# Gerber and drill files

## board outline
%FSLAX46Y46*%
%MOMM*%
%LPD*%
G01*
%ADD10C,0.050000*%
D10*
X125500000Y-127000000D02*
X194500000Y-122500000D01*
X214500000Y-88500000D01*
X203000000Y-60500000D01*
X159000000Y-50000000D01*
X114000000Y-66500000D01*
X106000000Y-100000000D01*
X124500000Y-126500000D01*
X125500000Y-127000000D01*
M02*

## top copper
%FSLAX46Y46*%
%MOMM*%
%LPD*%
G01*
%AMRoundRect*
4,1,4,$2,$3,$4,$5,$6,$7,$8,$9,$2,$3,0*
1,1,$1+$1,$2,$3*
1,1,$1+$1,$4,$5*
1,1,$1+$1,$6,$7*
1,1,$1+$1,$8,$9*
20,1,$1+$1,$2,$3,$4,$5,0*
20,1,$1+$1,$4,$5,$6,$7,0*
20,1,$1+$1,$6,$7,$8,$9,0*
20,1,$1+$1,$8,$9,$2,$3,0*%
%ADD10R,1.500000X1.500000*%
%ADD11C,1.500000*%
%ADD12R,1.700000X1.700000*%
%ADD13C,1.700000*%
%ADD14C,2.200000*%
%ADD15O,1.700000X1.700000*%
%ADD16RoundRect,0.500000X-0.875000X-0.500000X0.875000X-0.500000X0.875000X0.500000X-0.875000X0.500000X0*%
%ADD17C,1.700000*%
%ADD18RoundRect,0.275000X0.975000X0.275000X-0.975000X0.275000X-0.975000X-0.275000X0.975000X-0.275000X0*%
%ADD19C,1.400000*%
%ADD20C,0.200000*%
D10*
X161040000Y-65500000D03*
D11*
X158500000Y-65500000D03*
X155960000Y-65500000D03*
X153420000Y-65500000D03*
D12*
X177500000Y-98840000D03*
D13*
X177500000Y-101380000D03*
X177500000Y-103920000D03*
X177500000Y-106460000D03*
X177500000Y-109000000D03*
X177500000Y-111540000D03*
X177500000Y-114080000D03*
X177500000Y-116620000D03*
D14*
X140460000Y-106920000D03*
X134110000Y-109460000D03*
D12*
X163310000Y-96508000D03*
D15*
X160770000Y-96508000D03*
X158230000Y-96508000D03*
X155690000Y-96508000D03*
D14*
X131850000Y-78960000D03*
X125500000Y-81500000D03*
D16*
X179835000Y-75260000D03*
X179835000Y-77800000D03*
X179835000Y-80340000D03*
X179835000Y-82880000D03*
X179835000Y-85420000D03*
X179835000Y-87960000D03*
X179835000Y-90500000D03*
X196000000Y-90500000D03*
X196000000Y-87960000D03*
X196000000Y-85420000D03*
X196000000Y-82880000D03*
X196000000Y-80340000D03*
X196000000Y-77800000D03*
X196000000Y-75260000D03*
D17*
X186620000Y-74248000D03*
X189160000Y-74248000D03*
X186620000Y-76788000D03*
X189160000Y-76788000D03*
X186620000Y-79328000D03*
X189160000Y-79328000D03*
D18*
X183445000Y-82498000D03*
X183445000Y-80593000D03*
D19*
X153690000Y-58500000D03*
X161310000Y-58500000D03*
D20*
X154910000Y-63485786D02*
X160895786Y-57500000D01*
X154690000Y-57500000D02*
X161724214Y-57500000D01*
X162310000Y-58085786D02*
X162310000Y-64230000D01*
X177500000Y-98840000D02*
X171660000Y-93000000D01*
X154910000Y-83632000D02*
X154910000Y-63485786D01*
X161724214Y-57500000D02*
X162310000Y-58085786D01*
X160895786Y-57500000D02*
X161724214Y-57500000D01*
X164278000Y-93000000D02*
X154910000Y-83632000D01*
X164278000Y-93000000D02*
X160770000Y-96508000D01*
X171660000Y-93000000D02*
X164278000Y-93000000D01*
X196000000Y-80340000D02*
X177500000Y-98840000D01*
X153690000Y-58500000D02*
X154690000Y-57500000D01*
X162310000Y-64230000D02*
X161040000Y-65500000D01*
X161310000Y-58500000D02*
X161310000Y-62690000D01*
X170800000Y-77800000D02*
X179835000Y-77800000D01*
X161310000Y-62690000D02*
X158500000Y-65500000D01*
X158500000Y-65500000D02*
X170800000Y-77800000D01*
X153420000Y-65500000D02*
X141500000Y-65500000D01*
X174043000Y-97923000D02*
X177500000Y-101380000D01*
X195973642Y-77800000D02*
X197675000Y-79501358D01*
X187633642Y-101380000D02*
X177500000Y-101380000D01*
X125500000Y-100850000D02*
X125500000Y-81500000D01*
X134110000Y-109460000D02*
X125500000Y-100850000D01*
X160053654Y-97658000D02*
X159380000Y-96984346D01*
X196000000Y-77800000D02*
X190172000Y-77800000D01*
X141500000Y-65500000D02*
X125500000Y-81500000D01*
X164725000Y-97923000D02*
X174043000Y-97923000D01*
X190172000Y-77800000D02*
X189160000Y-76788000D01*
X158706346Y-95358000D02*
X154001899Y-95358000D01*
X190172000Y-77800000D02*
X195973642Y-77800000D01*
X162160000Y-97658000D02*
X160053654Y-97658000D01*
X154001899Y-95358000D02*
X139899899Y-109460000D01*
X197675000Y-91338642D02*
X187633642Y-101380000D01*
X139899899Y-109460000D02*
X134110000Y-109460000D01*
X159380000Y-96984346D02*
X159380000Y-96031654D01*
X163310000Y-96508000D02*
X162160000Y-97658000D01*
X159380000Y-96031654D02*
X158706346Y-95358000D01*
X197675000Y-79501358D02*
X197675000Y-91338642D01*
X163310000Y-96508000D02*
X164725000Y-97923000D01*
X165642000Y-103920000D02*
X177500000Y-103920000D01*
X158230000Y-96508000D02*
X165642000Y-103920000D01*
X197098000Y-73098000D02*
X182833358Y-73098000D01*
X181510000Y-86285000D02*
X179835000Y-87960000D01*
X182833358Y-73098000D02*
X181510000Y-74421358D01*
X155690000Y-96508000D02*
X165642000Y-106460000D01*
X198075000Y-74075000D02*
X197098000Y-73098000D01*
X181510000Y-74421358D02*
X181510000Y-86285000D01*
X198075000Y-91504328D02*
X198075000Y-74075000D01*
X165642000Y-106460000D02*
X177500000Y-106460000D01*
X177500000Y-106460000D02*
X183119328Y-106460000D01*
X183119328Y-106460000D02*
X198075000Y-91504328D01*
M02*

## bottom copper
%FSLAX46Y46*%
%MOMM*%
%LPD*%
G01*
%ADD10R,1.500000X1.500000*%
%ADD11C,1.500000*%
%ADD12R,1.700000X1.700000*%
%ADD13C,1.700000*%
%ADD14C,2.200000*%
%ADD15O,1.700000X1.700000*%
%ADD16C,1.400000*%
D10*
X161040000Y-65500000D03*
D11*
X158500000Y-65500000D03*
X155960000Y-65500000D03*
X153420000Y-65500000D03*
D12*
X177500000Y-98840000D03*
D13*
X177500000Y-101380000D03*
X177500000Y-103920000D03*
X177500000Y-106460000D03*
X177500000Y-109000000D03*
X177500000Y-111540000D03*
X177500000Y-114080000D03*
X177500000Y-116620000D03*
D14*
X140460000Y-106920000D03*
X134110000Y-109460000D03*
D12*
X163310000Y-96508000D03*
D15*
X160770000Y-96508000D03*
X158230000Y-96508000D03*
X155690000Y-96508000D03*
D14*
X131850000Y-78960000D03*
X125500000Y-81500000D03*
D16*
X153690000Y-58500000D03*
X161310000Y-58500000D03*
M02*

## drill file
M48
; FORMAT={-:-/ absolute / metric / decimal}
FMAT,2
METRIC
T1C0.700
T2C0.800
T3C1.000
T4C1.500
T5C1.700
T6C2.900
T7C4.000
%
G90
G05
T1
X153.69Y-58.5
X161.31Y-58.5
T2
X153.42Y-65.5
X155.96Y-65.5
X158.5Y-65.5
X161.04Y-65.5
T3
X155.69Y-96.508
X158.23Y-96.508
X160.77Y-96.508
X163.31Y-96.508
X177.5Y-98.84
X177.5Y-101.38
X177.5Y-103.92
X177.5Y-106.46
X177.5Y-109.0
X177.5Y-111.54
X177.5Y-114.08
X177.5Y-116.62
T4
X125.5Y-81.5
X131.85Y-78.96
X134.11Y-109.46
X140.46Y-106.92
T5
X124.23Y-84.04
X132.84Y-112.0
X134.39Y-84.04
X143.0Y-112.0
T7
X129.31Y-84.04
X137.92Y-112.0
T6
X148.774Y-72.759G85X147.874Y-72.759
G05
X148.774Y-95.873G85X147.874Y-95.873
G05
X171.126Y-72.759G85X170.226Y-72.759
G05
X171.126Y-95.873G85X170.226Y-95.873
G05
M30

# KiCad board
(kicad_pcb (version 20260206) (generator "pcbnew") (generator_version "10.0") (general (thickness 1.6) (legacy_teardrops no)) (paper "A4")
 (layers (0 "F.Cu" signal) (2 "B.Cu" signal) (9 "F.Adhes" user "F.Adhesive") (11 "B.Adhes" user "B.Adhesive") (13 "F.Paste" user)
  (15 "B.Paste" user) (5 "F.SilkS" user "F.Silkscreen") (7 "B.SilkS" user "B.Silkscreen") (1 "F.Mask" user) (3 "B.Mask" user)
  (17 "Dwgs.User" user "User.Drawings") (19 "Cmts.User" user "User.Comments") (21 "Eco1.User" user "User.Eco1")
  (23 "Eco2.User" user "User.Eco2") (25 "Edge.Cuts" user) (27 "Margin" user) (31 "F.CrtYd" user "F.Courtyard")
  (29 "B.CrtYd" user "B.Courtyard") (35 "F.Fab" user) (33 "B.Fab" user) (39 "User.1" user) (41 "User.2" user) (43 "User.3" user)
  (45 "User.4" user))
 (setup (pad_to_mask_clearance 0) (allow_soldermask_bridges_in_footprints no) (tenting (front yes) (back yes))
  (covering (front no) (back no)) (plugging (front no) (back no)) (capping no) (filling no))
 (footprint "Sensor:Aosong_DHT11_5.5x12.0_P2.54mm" (layer "F.Cu") (at 161.04 65.5 -90)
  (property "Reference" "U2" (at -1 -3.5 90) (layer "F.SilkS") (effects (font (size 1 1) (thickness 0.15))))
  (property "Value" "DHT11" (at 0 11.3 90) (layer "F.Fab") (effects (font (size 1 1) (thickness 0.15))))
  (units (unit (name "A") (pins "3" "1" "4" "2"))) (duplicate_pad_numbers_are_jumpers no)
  (pad "1" thru_hole rect (at 0 0 270) (size 1.5 1.5) (drill 0.8) (layers "*.Cu" "*.Mask") (remove_unused_layers no) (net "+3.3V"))
  (pad "2" thru_hole circle (at 0 2.54 270) (size 1.5 1.5) (drill 0.8) (layers "*.Cu" "*.Mask") (remove_unused_layers no)
   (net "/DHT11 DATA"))
  (pad "3" thru_hole circle (at 0 5.08 270) (size 1.5 1.5) (drill 0.8) (layers "*.Cu" "*.Mask") (remove_unused_layers no)
   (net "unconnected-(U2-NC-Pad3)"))
  (pad "4" thru_hole circle (at 0 7.62 270) (size 1.5 1.5) (drill 0.8) (layers "*.Cu" "*.Mask") (remove_unused_layers no) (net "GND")))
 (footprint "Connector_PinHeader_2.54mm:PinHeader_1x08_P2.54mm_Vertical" (layer "F.Cu") (at 177.5 98.84)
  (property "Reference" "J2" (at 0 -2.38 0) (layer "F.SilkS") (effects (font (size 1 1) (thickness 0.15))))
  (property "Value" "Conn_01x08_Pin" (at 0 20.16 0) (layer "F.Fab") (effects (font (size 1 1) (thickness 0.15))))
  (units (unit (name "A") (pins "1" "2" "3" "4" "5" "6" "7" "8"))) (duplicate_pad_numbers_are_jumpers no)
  (pad "1" thru_hole rect (at 0 0) (size 1.7 1.7) (drill 1) (layers "*.Cu" "*.Mask") (remove_unused_layers no) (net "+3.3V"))
  (pad "2" thru_hole circle (at 0 2.54) (size 1.7 1.7) (drill 1) (layers "*.Cu" "*.Mask") (remove_unused_layers no) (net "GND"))
  (pad "3" thru_hole circle (at 0 5.08) (size 1.7 1.7) (drill 1) (layers "*.Cu" "*.Mask") (remove_unused_layers no) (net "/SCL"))
  (pad "4" thru_hole circle (at 0 7.62) (size 1.7 1.7) (drill 1) (layers "*.Cu" "*.Mask") (remove_unused_layers no) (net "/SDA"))
  (pad "5" thru_hole circle (at 0 10.16) (size 1.7 1.7) (drill 1) (layers "*.Cu" "*.Mask") (remove_unused_layers no)
   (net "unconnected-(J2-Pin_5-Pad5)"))
  (pad "6" thru_hole circle (at 0 12.7) (size 1.7 1.7) (drill 1) (layers "*.Cu" "*.Mask") (remove_unused_layers no)
   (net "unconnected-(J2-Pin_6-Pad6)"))
  (pad "7" thru_hole circle (at 0 15.24) (size 1.7 1.7) (drill 1) (layers "*.Cu" "*.Mask") (remove_unused_layers no)
   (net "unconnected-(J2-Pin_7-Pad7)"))
  (pad "8" thru_hole circle (at 0 17.78) (size 1.7 1.7) (drill 1) (layers "*.Cu" "*.Mask") (remove_unused_layers no)
   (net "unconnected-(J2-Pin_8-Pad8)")))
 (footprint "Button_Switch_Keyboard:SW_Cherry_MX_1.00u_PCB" (layer "F.Cu") (at 140.46 106.92)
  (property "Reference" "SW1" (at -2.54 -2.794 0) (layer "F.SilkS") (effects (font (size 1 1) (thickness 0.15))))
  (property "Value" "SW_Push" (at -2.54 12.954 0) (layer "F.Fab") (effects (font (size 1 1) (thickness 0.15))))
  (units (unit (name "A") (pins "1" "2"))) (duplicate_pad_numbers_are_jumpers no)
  (pad "" np_thru_hole circle (at -7.62 5.08) (size 1.7 1.7) (drill 1.7) (layers "*.Cu" "*.Mask"))
  (pad "" np_thru_hole circle (at -2.54 5.08) (size 4 4) (drill 4) (layers "*.Cu" "*.Mask"))
  (pad "" np_thru_hole circle (at 2.54 5.08) (size 1.7 1.7) (drill 1.7) (layers "*.Cu" "*.Mask"))
  (pad "1" thru_hole circle (at 0 0) (size 2.2 2.2) (drill 1.5) (layers "*.Cu" "*.Mask") (remove_unused_layers no) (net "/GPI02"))
  (pad "2" thru_hole circle (at -6.35 2.54) (size 2.2 2.2) (drill 1.5) (layers "*.Cu" "*.Mask") (remove_unused_layers no) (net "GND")))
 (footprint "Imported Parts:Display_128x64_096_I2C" (layer "F.Cu") (at 159.5 96.508 180)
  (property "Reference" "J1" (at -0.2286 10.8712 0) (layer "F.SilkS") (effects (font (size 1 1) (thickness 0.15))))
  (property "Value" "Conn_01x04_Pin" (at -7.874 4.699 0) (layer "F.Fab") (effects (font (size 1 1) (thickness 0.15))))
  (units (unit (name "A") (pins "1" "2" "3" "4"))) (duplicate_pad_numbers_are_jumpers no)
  (pad "" np_thru_hole oval (at -11.176 0.635 180) (size 3.8 2.9) (drill oval 3.8 2.9) (layers "*.Cu" "*.Mask"))
  (pad "" np_thru_hole oval (at -11.176 23.749 180) (size 3.8 2.9) (drill oval 3.8 2.9) (layers "*.Cu" "*.Mask"))
  (pad "" np_thru_hole oval (at 11.176 0.635 180) (size 3.8 2.9) (drill oval 3.8 2.9) (layers "*.Cu" "*.Mask"))
  (pad "" np_thru_hole oval (at 11.176 23.749 180) (size 3.8 2.9) (drill oval 3.8 2.9) (layers "*.Cu" "*.Mask"))
  (pad "1" thru_hole rect (at -3.81 0 270) (size 1.7 1.7) (drill 1) (layers "*.Cu" "*.Mask") (remove_unused_layers no) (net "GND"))
  (pad "2" thru_hole oval (at -1.27 0 270) (size 1.7 1.7) (drill 1) (layers "*.Cu" "*.Mask") (remove_unused_layers no) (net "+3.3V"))
  (pad "3" thru_hole oval (at 1.27 0 270) (size 1.7 1.7) (drill 1) (layers "*.Cu" "*.Mask") (remove_unused_layers no) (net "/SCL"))
  (pad "4" thru_hole oval (at 3.81 0 270) (size 1.7 1.7) (drill 1) (layers "*.Cu" "*.Mask") (remove_unused_layers no) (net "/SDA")))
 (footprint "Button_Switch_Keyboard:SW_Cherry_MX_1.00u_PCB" (layer "F.Cu") (at 131.85 78.96)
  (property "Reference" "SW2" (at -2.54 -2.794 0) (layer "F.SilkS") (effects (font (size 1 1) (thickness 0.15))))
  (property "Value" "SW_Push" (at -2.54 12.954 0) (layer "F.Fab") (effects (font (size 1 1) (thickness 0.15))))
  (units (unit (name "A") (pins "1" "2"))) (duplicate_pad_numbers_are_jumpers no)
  (pad "" np_thru_hole circle (at -7.62 5.08) (size 1.7 1.7) (drill 1.7) (layers "*.Cu" "*.Mask"))
  (pad "" np_thru_hole circle (at -2.54 5.08) (size 4 4) (drill 4) (layers "*.Cu" "*.Mask"))
  (pad "" np_thru_hole circle (at 2.54 5.08) (size 1.7 1.7) (drill 1.7) (layers "*.Cu" "*.Mask"))
  (pad "1" thru_hole circle (at 0 0) (size 2.2 2.2) (drill 1.5) (layers "*.Cu" "*.Mask") (remove_unused_layers no) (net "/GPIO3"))
  (pad "2" thru_hole circle (at -6.35 2.54) (size 2.2 2.2) (drill 1.5) (layers "*.Cu" "*.Mask") (remove_unused_layers no) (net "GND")))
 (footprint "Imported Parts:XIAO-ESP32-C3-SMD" (layer "F.Cu") (at 179 93.38)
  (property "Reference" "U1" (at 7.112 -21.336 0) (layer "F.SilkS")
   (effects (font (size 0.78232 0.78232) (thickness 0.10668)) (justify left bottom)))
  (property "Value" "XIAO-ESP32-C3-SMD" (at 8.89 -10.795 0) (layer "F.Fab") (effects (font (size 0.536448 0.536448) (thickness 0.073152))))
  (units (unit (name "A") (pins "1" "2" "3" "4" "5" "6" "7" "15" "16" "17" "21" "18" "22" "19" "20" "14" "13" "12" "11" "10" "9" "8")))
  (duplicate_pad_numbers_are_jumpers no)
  (pad "1" smd roundrect (at 0.835 -18.12) (size 2.75 2) (layers "F.Cu" "F.Mask" "F.Paste") (roundrect_rratio 0.25)
   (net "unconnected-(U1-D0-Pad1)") (solder_mask_margin 0.0508) (thermal_bridge_angle 45))
  (pad "2" smd roundrect (at 0.835 -15.58) (size 2.75 2) (layers "F.Cu" "F.Mask" "F.Paste") (roundrect_rratio 0.25) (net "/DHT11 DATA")
   (solder_mask_margin 0.0508) (thermal_bridge_angle 45))
  (pad "3" smd roundrect (at 0.835 -13.04) (size 2.75 2) (layers "F.Cu" "F.Mask" "F.Paste") (roundrect_rratio 0.25) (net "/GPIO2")
   (solder_mask_margin 0.0508) (thermal_bridge_angle 45))
  (pad "4" smd roundrect (at 0.835 -10.5) (size 2.75 2) (layers "F.Cu" "F.Mask" "F.Paste") (roundrect_rratio 0.25) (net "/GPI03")
   (solder_mask_margin 0.0508) (thermal_bridge_angle 45))
  (pad "5" smd roundrect (at 0.835 -7.96) (size 2.75 2) (layers "F.Cu" "F.Mask" "F.Paste") (roundrect_rratio 0.25) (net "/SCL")
   (solder_mask_margin 0.0508) (thermal_bridge_angle 45))
  (pad "6" smd roundrect (at 0.835 -5.42) (size 2.75 2) (layers "F.Cu" "F.Mask" "F.Paste") (roundrect_rratio 0.25) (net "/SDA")
   (solder_mask_margin 0.0508) (thermal_bridge_angle 45))
  (pad "7" smd roundrect (at 0.835 -2.88) (size 2.75 2) (layers "F.Cu" "F.Mask" "F.Paste") (roundrect_rratio 0.25)
   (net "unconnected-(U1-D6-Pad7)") (solder_mask_margin 0.0508) (thermal_bridge_angle 45))
  (pad "8" smd roundrect (at 17 -2.88) (size 2.75 2) (layers "F.Cu" "F.Mask" "F.Paste") (roundrect_rratio 0.25)
   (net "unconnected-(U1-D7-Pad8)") (solder_mask_margin 0.0508) (thermal_bridge_angle 45))
  (pad "9" smd roundrect (at 17 -5.42) (size 2.75 2) (layers "F.Cu" "F.Mask" "F.Paste") (roundrect_rratio 0.25)
   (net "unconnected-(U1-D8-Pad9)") (solder_mask_margin 0.0508) (thermal_bridge_angle 45))
  (pad "10" smd roundrect (at 17 -7.96) (size 2.75 2) (layers "F.Cu" "F.Mask" "F.Paste") (roundrect_rratio 0.25)
   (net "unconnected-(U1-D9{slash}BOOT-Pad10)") (solder_mask_margin 0.0508) (thermal_bridge_angle 45))
  (pad "11" smd roundrect (at 17 -10.5) (size 2.75 2) (layers "F.Cu" "F.Mask" "F.Paste") (roundrect_rratio 0.25)
   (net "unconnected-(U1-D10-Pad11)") (solder_mask_margin 0.0508) (thermal_bridge_angle 45))
  (pad "12" smd roundrect (at 17 -13.04) (size 2.75 2) (layers "F.Cu" "F.Mask" "F.Paste") (roundrect_rratio 0.25) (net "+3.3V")
   (solder_mask_margin 0.0508) (thermal_bridge_angle 45))
  (pad "13" smd roundrect (at 17 -15.58) (size 2.75 2) (layers "F.Cu" "F.Mask" "F.Paste") (roundrect_rratio 0.25) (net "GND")
   (solder_mask_margin 0.0508) (thermal_bridge_angle 45))
  (pad "14" smd roundrect (at 17 -18.12) (size 2.75 2) (layers "F.Cu" "F.Mask" "F.Paste") (roundrect_rratio 0.25) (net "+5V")
   (solder_mask_margin 0.0508) (thermal_bridge_angle 45))
  (pad "15" smd circle (at 7.62 -19.132) (size 1.7 1.7) (layers "F.Cu" "F.Mask" "F.Paste") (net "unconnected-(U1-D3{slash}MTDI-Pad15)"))
  (pad "16" smd circle (at 10.16 -19.132) (size 1.7 1.7) (layers "F.Cu" "F.Mask" "F.Paste") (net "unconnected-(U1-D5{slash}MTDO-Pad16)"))
  (pad "17" smd circle (at 7.62 -16.592) (size 1.7 1.7) (layers "F.Cu" "F.Mask" "F.Paste") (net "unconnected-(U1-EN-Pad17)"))
  (pad "18" smd circle (at 10.16 -16.592) (size 1.7 1.7) (layers "F.Cu" "F.Mask" "F.Paste") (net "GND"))
  (pad "19" smd circle (at 7.62 -14.052) (size 1.7 1.7) (layers "F.Cu" "F.Mask" "F.Paste") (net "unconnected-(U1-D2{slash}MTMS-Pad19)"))
  (pad "20" smd circle (at 10.16 -14.052) (size 1.7 1.7) (layers "F.Cu" "F.Mask" "F.Paste") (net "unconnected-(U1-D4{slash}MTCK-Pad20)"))
  (pad "21" smd roundrect (at 4.445 -10.882 180) (size 2.5 1.1) (layers "F.Cu" "F.Mask" "F.Paste") (roundrect_rratio 0.25)
   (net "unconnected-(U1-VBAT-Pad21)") (thermal_bridge_angle 45))
  (pad "22" smd roundrect (at 4.445 -12.787 180) (size 2.5 1.1) (layers "F.Cu" "F.Mask" "F.Paste") (roundrect_rratio 0.25)
   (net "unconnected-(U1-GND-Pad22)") (thermal_bridge_angle 45)))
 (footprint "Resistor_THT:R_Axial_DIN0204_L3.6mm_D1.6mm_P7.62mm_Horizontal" (layer "F.Cu") (at 153.69 58.5)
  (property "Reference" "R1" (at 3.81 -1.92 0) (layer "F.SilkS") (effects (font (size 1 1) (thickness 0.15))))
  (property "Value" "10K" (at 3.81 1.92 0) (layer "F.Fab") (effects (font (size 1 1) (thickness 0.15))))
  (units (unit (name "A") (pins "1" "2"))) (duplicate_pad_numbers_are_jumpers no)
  (pad "1" thru_hole circle (at 0 0) (size 1.4 1.4) (drill 0.7) (layers "*.Cu" "*.Mask") (remove_unused_layers no) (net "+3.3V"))
  (pad "2" thru_hole circle (at 7.62 0) (size 1.4 1.4) (drill 0.7) (layers "*.Cu" "*.Mask") (remove_unused_layers no) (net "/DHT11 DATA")))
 (gr_poly
  (pts (xy 125.5 127) (xy 194.5 122.5) (xy 214.5 88.5) (xy 203 60.5) (xy 159 50) (xy 114 66.5) (xy 106 100) (xy 124.5 126.5))
  (stroke (width 0.05) (type solid)) (fill no) (layer "Edge.Cuts"))
 (segment (start 154.91 63.485786) (end 160.895786 57.5) (width 0.2) (layer "F.Cu") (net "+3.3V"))
 (segment (start 154.69 57.5) (end 161.724214 57.5) (width 0.2) (layer "F.Cu") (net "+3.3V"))
 (segment (start 162.31 58.085786) (end 162.31 64.23) (width 0.2) (layer "F.Cu") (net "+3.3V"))
 (segment (start 177.5 98.84) (end 171.66 93) (width 0.2) (layer "F.Cu") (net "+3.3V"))
 (segment (start 154.91 83.632) (end 154.91 63.485786) (width 0.2) (layer "F.Cu") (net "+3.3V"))
 (segment (start 161.724214 57.5) (end 162.31 58.085786) (width 0.2) (layer "F.Cu") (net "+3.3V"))
 (segment (start 160.895786 57.5) (end 161.724214 57.5) (width 0.2) (layer "F.Cu") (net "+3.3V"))
 (segment (start 164.278 93) (end 154.91 83.632) (width 0.2) (layer "F.Cu") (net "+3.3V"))
 (segment (start 164.278 93) (end 160.77 96.508) (width 0.2) (layer "F.Cu") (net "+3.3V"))
 (segment (start 171.66 93) (end 164.278 93) (width 0.2) (layer "F.Cu") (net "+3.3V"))
 (segment (start 196 80.34) (end 177.5 98.84) (width 0.2) (layer "F.Cu") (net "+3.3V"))
 (segment (start 153.69 58.5) (end 154.69 57.5) (width 0.2) (layer "F.Cu") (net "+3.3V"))
 (segment (start 162.31 64.23) (end 161.04 65.5) (width 0.2) (layer "F.Cu") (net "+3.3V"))
 (segment (start 161.31 58.5) (end 161.31 62.69) (width 0.2) (layer "F.Cu") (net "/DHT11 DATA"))
 (segment (start 170.8 77.8) (end 179.835 77.8) (width 0.2) (layer "F.Cu") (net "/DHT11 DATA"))
 (segment (start 161.31 62.69) (end 158.5 65.5) (width 0.2) (layer "F.Cu") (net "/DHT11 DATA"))
 (segment (start 158.5 65.5) (end 170.8 77.8) (width 0.2) (layer "F.Cu") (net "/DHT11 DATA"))
 (segment (start 153.42 65.5) (end 141.5 65.5) (width 0.2) (layer "F.Cu") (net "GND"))
 (segment (start 174.043 97.923) (end 177.5 101.38) (width 0.2) (layer "F.Cu") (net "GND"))
 (segment (start 195.973642 77.8) (end 197.675 79.501358) (width 0.2) (layer "F.Cu") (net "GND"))
 (segment (start 187.633642 101.38) (end 177.5 101.38) (width 0.2) (layer "F.Cu") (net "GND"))
 (segment (start 125.5 100.85) (end 125.5 81.5) (width 0.2) (layer "F.Cu") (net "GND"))
 (segment (start 134.11 109.46) (end 125.5 100.85) (width 0.2) (layer "F.Cu") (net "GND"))
 (segment (start 160.053654 97.658) (end 159.38 96.984346) (width 0.2) (layer "F.Cu") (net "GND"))
 (segment (start 196 77.8) (end 190.172 77.8) (width 0.2) (layer "F.Cu") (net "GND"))
 (segment (start 141.5 65.5) (end 125.5 81.5) (width 0.2) (layer "F.Cu") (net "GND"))
 (segment (start 164.725 97.923) (end 174.043 97.923) (width 0.2) (layer "F.Cu") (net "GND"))
 (segment (start 190.172 77.8) (end 189.16 76.788) (width 0.2) (layer "F.Cu") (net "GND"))
 (segment (start 158.706346 95.358) (end 154.001899 95.358) (width 0.2) (layer "F.Cu") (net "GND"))
 (segment (start 190.172 77.8) (end 195.973642 77.8) (width 0.2) (layer "F.Cu") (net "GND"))
 (segment (start 162.16 97.658) (end 160.053654 97.658) (width 0.2) (layer "F.Cu") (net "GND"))
 (segment (start 154.001899 95.358) (end 139.899899 109.46) (width 0.2) (layer "F.Cu") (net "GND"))
 (segment (start 197.675 91.338642) (end 187.633642 101.38) (width 0.2) (layer "F.Cu") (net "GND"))
 (segment (start 139.899899 109.46) (end 134.11 109.46) (width 0.2) (layer "F.Cu") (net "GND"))
 (segment (start 159.38 96.984346) (end 159.38 96.031654) (width 0.2) (layer "F.Cu") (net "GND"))
 (segment (start 163.31 96.508) (end 162.16 97.658) (width 0.2) (layer "F.Cu") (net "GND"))
 (segment (start 159.38 96.031654) (end 158.706346 95.358) (width 0.2) (layer "F.Cu") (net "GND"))
 (segment (start 197.675 79.501358) (end 197.675 91.338642) (width 0.2) (layer "F.Cu") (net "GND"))
 (segment (start 163.31 96.508) (end 164.725 97.923) (width 0.2) (layer "F.Cu") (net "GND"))
 (segment (start 165.642 103.92) (end 177.5 103.92) (width 0.2) (layer "F.Cu") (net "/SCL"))
 (segment (start 158.23 96.508) (end 165.642 103.92) (width 0.2) (layer "F.Cu") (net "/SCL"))
 (segment (start 197.098 73.098) (end 182.833358 73.098) (width 0.2) (layer "F.Cu") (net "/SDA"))
 (segment (start 181.51 86.285) (end 179.835 87.96) (width 0.2) (layer "F.Cu") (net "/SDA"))
 (segment (start 182.833358 73.098) (end 181.51 74.421358) (width 0.2) (layer "F.Cu") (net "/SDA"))
 (segment (start 155.69 96.508) (end 165.642 106.46) (width 0.2) (layer "F.Cu") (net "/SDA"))
 (segment (start 198.075 74.075) (end 197.098 73.098) (width 0.2) (layer "F.Cu") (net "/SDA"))
 (segment (start 181.51 74.421358) (end 181.51 86.285) (width 0.2) (layer "F.Cu") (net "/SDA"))
 (segment (start 198.075 91.504328) (end 198.075 74.075) (width 0.2) (layer "F.Cu") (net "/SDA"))
 (segment (start 165.642 106.46) (end 177.5 106.46) (width 0.2) (layer "F.Cu") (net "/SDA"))
 (segment (start 177.5 106.46) (end 183.119328 106.46) (width 0.2) (layer "F.Cu") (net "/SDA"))
 (segment (start 183.119328 106.46) (end 198.075 91.504328) (width 0.2) (layer "F.Cu") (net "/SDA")))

